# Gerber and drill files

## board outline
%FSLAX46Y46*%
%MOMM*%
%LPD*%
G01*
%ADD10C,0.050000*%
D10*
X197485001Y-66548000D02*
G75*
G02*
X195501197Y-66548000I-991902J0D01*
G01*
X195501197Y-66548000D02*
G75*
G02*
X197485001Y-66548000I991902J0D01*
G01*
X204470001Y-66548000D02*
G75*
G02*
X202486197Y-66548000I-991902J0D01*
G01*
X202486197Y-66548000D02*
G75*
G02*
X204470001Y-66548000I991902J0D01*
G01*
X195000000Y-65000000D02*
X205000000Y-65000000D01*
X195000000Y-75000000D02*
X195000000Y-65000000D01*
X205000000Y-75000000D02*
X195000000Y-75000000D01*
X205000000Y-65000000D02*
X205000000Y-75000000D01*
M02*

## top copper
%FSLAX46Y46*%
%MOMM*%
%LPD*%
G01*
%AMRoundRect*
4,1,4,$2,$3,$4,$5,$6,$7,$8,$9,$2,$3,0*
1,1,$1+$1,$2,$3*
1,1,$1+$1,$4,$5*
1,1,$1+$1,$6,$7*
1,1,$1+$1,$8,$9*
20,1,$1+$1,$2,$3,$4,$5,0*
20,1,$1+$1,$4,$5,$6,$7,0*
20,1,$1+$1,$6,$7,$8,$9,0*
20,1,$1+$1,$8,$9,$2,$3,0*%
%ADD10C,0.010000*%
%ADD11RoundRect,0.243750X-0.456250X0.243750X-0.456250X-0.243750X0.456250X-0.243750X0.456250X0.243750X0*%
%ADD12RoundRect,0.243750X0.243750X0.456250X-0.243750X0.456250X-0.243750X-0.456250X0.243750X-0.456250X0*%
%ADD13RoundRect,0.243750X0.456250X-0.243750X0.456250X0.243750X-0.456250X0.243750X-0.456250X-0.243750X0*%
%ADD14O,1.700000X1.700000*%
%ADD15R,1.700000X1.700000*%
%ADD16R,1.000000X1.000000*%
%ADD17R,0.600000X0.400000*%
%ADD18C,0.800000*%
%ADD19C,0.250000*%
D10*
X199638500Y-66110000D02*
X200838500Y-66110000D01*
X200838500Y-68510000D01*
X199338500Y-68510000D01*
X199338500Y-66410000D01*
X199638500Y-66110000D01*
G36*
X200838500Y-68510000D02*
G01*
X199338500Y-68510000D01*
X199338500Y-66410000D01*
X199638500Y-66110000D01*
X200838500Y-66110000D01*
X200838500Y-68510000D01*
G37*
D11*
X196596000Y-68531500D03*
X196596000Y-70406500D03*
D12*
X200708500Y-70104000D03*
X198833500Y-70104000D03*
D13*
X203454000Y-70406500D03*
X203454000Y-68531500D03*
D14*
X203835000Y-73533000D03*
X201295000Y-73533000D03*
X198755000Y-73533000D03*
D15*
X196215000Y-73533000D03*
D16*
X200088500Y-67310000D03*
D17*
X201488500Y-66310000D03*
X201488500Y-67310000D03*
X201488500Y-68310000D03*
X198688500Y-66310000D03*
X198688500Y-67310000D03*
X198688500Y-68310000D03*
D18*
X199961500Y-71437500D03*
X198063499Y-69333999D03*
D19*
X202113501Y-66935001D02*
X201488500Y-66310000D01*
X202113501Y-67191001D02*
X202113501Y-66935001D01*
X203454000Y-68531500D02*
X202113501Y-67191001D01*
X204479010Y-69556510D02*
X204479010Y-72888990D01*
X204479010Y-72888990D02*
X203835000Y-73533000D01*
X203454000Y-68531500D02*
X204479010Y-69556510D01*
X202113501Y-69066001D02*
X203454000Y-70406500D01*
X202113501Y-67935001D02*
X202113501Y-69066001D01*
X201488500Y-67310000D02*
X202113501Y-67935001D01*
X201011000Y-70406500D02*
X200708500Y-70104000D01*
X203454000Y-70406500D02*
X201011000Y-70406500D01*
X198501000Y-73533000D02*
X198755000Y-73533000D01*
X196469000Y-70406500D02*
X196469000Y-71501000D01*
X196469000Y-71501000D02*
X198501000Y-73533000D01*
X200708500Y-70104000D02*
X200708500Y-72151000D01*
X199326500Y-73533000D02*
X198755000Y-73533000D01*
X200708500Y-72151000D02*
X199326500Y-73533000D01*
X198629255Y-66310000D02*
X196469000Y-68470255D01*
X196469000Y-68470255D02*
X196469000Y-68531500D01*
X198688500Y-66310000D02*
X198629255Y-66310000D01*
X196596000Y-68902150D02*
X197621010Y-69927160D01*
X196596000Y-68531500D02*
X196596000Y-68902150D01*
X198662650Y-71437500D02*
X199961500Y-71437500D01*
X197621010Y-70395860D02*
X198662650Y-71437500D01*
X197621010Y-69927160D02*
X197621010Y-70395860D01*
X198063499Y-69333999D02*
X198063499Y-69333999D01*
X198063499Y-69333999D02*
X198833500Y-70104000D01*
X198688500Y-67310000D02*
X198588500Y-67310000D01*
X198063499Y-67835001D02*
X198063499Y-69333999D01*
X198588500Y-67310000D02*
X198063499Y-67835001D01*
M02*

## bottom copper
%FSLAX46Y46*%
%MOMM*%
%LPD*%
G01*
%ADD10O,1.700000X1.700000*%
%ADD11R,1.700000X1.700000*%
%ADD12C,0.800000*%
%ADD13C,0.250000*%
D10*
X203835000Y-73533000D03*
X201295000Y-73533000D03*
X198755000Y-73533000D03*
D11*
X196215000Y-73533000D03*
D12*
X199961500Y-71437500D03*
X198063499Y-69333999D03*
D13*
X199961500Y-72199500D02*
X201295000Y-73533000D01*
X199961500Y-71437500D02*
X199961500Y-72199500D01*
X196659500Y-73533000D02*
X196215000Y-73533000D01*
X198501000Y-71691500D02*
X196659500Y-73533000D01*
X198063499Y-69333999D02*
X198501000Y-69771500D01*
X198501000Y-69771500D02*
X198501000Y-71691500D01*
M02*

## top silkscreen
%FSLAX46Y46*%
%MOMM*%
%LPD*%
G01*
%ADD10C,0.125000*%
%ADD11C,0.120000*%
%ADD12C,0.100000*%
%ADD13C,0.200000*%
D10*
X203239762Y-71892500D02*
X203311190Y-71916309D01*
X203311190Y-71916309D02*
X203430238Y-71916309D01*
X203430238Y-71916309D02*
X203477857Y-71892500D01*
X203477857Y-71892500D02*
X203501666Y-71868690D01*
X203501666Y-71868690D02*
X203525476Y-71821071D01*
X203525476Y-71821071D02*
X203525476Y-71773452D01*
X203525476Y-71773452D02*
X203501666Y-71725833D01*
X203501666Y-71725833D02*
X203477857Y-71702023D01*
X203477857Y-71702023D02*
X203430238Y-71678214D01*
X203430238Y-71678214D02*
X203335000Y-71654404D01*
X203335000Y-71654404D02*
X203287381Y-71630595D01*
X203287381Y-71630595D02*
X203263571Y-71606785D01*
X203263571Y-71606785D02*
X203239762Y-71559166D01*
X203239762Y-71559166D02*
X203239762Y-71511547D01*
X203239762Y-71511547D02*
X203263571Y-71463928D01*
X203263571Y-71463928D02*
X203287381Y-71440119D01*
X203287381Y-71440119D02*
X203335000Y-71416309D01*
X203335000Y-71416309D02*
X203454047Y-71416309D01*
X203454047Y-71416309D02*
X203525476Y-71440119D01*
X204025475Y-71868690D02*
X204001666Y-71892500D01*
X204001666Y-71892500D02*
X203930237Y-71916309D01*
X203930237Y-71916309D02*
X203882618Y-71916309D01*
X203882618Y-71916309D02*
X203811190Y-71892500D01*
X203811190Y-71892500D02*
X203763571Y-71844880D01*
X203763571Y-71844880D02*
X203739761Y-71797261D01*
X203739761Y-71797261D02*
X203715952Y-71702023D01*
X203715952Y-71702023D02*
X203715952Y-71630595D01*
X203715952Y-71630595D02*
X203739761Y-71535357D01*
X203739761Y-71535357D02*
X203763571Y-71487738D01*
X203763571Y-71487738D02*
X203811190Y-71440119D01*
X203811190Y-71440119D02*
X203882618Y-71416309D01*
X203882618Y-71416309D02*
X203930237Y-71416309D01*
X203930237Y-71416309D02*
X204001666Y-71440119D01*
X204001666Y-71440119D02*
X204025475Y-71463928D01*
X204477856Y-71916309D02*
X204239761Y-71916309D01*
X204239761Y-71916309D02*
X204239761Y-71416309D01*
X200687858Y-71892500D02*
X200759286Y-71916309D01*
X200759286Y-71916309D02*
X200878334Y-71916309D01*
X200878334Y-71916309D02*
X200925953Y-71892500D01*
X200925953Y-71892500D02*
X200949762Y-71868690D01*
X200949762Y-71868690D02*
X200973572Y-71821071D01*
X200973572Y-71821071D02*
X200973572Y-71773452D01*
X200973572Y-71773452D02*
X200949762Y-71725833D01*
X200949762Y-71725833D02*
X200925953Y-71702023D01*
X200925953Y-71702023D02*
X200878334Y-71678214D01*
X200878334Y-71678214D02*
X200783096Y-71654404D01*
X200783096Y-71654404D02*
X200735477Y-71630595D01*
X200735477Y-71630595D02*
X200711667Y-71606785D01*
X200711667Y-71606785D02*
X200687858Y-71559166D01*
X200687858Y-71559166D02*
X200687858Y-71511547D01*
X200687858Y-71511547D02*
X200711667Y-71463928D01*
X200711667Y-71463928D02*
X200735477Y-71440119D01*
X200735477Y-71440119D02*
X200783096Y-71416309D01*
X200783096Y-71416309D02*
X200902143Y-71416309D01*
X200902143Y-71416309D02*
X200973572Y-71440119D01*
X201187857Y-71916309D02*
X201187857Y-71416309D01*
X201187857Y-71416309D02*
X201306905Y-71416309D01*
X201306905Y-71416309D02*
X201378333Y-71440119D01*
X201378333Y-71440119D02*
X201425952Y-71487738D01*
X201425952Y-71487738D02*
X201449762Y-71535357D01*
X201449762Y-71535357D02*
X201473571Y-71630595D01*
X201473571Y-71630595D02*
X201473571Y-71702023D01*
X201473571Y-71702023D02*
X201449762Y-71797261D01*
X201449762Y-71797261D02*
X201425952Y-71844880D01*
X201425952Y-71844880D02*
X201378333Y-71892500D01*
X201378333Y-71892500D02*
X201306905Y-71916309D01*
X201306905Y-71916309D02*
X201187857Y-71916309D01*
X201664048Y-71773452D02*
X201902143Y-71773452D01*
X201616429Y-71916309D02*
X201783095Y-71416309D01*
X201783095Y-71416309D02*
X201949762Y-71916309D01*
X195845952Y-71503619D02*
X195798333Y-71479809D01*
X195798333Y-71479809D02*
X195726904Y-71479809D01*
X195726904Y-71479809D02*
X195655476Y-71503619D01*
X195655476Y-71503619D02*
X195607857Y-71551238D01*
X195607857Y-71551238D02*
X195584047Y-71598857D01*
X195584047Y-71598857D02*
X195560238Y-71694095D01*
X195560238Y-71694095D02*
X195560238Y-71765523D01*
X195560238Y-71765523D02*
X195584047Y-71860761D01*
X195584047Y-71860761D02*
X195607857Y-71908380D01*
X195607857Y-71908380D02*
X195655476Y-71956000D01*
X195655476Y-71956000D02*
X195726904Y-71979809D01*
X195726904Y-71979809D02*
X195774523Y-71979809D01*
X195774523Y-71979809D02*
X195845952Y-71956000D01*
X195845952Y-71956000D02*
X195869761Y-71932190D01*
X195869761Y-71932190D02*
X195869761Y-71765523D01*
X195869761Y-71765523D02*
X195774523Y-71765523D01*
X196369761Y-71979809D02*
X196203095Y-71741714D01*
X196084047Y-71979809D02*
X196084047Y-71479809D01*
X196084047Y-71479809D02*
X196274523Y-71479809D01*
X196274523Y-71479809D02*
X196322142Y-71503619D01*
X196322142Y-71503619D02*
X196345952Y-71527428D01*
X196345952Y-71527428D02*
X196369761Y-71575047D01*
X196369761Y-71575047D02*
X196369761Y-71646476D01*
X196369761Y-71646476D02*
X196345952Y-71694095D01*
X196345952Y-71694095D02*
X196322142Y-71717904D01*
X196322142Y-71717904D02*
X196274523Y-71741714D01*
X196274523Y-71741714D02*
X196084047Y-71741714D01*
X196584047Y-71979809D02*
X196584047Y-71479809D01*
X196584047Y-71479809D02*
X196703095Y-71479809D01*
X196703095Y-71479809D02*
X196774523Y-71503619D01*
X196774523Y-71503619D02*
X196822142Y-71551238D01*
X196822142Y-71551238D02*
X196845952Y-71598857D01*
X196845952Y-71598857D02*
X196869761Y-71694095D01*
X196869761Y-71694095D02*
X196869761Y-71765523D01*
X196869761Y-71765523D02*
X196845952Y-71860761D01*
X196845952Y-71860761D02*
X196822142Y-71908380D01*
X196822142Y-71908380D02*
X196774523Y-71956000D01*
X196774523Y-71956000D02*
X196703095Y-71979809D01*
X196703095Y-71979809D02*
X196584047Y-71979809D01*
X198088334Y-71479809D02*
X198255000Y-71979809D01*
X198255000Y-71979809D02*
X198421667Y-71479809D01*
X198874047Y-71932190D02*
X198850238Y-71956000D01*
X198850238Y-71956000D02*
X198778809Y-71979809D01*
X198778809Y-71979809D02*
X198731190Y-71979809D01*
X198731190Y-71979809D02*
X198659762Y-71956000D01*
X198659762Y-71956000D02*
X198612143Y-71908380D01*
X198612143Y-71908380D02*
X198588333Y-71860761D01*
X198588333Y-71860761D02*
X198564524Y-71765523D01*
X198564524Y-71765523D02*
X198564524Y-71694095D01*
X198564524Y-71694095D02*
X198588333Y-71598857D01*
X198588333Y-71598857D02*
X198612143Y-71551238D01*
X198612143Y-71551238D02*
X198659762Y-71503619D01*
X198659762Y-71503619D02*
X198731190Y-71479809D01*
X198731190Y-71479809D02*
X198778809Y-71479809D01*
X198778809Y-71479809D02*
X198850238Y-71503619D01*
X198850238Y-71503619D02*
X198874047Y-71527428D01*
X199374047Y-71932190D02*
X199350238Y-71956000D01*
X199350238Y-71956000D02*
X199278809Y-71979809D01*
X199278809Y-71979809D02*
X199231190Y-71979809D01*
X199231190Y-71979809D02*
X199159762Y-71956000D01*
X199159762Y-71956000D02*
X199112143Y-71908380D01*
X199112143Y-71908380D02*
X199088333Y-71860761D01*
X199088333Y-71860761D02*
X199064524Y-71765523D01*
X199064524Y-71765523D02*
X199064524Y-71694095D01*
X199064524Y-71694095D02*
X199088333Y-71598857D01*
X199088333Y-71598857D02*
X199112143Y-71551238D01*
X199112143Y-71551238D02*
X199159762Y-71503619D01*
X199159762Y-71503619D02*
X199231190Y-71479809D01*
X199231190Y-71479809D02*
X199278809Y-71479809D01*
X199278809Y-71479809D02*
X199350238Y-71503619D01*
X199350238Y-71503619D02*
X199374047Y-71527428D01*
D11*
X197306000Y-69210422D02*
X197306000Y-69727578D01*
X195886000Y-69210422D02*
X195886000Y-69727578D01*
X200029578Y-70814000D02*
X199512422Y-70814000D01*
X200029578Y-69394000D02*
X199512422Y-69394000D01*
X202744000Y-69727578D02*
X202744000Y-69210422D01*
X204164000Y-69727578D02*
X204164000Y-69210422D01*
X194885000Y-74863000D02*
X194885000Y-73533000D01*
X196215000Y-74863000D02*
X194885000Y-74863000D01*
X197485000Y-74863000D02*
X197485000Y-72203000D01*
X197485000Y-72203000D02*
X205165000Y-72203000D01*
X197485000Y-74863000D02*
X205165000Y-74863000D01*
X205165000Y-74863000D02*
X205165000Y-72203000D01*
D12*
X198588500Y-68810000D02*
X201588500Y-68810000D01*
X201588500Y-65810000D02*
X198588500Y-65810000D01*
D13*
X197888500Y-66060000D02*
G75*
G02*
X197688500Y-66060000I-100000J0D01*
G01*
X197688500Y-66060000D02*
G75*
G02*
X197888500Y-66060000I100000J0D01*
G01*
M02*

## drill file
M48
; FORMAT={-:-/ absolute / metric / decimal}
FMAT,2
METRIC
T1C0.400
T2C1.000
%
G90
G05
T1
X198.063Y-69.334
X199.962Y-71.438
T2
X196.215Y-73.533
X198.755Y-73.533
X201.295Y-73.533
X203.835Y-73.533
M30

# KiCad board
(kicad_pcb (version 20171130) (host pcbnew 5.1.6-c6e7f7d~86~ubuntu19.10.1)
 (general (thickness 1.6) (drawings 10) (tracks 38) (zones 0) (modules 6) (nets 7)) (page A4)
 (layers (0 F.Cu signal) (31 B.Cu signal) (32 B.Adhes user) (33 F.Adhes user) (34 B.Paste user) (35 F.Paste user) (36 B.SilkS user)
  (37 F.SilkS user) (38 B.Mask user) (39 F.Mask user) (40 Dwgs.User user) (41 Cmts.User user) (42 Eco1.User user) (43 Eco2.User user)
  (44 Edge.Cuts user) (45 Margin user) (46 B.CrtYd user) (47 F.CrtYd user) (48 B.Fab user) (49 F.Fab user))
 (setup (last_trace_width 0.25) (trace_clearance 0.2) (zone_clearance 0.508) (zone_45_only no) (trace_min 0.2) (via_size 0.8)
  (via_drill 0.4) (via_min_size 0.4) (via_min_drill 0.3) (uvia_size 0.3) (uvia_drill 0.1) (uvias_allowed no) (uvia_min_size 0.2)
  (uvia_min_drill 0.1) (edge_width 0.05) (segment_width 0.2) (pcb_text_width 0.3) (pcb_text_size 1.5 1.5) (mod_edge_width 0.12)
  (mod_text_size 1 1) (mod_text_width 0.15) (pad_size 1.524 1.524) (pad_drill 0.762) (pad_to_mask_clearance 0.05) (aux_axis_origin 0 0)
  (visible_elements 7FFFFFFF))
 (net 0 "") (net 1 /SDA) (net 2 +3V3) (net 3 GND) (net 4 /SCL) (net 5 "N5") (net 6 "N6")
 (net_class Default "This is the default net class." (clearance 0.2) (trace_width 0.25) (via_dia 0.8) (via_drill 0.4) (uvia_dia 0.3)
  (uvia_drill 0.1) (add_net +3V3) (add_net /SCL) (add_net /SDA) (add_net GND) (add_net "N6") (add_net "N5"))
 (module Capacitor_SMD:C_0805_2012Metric (layer F.Cu) (at 196.596 69.469 270)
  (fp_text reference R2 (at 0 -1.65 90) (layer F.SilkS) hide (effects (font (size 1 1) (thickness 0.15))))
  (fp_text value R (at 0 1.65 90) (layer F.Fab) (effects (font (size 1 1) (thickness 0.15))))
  (fp_line (start -0.258578 -0.71) (end 0.258578 -0.71) (layer F.SilkS) (width 0.12))
  (fp_line (start -0.258578 0.71) (end 0.258578 0.71) (layer F.SilkS) (width 0.12))
  (pad 1 smd roundrect (at -0.9375 0 270) (size 0.975 1.4) (layers F.Cu F.Paste F.Mask) (roundrect_rratio 0.25) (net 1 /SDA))
  (pad 2 smd roundrect (at 0.9375 0 270) (size 0.975 1.4) (layers F.Cu F.Paste F.Mask) (roundrect_rratio 0.25) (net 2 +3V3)))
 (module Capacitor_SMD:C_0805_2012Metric (layer F.Cu) (at 199.771 70.104 180)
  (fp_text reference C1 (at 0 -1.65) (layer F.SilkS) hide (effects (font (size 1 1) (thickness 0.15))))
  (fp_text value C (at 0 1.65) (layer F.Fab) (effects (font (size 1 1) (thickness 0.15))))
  (fp_line (start -0.258578 -0.71) (end 0.258578 -0.71) (layer F.SilkS) (width 0.12))
  (fp_line (start -0.258578 0.71) (end 0.258578 0.71) (layer F.SilkS) (width 0.12))
  (pad 1 smd roundrect (at -0.9375 0 180) (size 0.975 1.4) (layers F.Cu F.Paste F.Mask) (roundrect_rratio 0.25) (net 2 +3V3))
  (pad 2 smd roundrect (at 0.9375 0 180) (size 0.975 1.4) (layers F.Cu F.Paste F.Mask) (roundrect_rratio 0.25) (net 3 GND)))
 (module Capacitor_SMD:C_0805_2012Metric (layer F.Cu) (at 203.454 69.469 90)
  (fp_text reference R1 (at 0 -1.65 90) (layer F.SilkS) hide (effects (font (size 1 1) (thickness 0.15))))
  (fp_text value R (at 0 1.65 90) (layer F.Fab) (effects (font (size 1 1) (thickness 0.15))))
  (fp_line (start -0.258578 -0.71) (end 0.258578 -0.71) (layer F.SilkS) (width 0.12))
  (fp_line (start -0.258578 0.71) (end 0.258578 0.71) (layer F.SilkS) (width 0.12))
  (pad 1 smd roundrect (at -0.9375 0 90) (size 0.975 1.4) (layers F.Cu F.Paste F.Mask) (roundrect_rratio 0.25) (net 2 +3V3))
  (pad 2 smd roundrect (at 0.9375 0 90) (size 0.975 1.4) (layers F.Cu F.Paste F.Mask) (roundrect_rratio 0.25) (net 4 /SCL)))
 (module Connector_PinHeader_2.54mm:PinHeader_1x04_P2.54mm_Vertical (layer F.Cu) (at 196.215 73.533 90)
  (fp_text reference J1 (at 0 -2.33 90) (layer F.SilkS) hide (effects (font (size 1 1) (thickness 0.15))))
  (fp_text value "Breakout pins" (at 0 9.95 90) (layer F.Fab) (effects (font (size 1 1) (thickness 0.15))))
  (fp_line (start -1.33 -1.33) (end 0 -1.33) (layer F.SilkS) (width 0.12))
  (fp_line (start -1.33 0) (end -1.33 -1.33) (layer F.SilkS) (width 0.12))
  (fp_line (start -1.33 1.27) (end 1.33 1.27) (layer F.SilkS) (width 0.12))
  (fp_line (start 1.33 1.27) (end 1.33 8.95) (layer F.SilkS) (width 0.12))
  (fp_line (start -1.33 1.27) (end -1.33 8.95) (layer F.SilkS) (width 0.12))
  (fp_line (start -1.33 8.95) (end 1.33 8.95) (layer F.SilkS) (width 0.12))
  (pad 4 thru_hole oval (at 0 7.62 90) (size 1.7 1.7) (drill 1) (layers *.Cu *.Mask) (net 4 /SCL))
  (pad 3 thru_hole oval (at 0 5.08 90) (size 1.7 1.7) (drill 1) (layers *.Cu *.Mask) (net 1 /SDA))
  (pad 2 thru_hole oval (at 0 2.54 90) (size 1.7 1.7) (drill 1) (layers *.Cu *.Mask) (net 2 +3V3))
  (pad 1 thru_hole rect (at 0 0 90) (size 1.7 1.7) (drill 1) (layers *.Cu *.Mask) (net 3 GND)))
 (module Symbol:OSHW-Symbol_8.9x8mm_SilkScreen (layer B.Cu) (at 200.0885 70.739 180)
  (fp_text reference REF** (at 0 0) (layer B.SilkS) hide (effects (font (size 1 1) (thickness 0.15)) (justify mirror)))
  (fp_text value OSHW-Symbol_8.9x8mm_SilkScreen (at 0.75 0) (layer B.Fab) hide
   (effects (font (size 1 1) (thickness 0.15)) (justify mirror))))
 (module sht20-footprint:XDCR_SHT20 (layer F.Cu) (at 200.0885 67.31)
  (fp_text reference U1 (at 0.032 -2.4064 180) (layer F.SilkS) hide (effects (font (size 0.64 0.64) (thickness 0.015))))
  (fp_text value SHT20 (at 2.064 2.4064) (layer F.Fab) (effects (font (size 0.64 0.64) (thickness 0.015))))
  (fp_line (start -1.5 1.5) (end 1.5 1.5) (layer F.SilkS) (width 0.1))
  (fp_line (start 1.5 -1.5) (end -1.5 -1.5) (layer F.SilkS) (width 0.1))
  (fp_circle (center -2.3 -1.25) (end -2.2 -1.25) (layer F.SilkS) (width 0.2))
  (fp_poly (pts (xy -0.45 -1.2) (xy 0.75 -1.2) (xy 0.75 1.2) (xy -0.75 1.2) (xy -0.75 -0.9)) (layer F.Cu) (width 0.01))
  (pad 7 smd rect (at 0 0) (size 1 1) (layers F.Cu) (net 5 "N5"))
  (pad 6 smd rect (at 1.4 -1) (size 0.6 0.4) (layers F.Cu F.Mask) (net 4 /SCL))
  (pad 5 smd rect (at 1.4 0) (size 0.6 0.4) (layers F.Cu F.Mask) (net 2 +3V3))
  (pad 4 smd rect (at 1.4 1) (size 0.6 0.4) (layers F.Cu F.Mask) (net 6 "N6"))
  (pad 1 smd rect (at -1.4 -1) (size 0.6 0.4) (layers F.Cu F.Mask) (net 1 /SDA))
  (pad 2 smd rect (at -1.4 0) (size 0.6 0.4) (layers F.Cu F.Mask) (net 3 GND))
  (pad 3 smd rect (at -1.4 1) (size 0.6 0.4) (layers F.Cu F.Mask) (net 6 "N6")))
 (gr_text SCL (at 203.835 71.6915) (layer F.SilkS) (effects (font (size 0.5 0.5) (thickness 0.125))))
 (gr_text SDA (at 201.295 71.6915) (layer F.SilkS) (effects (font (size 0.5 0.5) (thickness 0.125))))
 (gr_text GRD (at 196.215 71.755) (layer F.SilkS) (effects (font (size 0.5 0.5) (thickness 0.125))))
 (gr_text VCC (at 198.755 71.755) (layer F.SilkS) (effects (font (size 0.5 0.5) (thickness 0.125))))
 (gr_circle (center 196.493099 66.548) (end 197.255099 67.183) (layer Edge.Cuts) (width 0.05))
 (gr_circle (center 203.478099 66.548) (end 204.240099 67.183) (layer Edge.Cuts) (width 0.05))
 (gr_line (start 195 65) (end 205 65) (layer Edge.Cuts) (width 0.05))
 (gr_line (start 195 75) (end 195 65) (layer Edge.Cuts) (width 0.05))
 (gr_line (start 205 75) (end 195 75) (layer Edge.Cuts) (width 0.05))
 (gr_line (start 205 65) (end 205 75) (layer Edge.Cuts) (width 0.05))
 (segment (start 202.113501 66.935001) (end 201.4885 66.31) (width 0.25) (layer F.Cu) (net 4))
 (segment (start 202.113501 67.191001) (end 202.113501 66.935001) (width 0.25) (layer F.Cu) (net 4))
 (segment (start 203.454 68.5315) (end 202.113501 67.191001) (width 0.25) (layer F.Cu) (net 4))
 (segment (start 204.47901 69.55651) (end 204.47901 72.88899) (width 0.25) (layer F.Cu) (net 4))
 (segment (start 204.47901 72.88899) (end 203.835 73.533) (width 0.25) (layer F.Cu) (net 4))
 (segment (start 203.454 68.5315) (end 204.47901 69.55651) (width 0.25) (layer F.Cu) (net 4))
 (segment (start 202.113501 69.066001) (end 203.454 70.4065) (width 0.25) (layer F.Cu) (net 2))
 (segment (start 202.113501 67.935001) (end 202.113501 69.066001) (width 0.25) (layer F.Cu) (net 2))
 (segment (start 201.4885 67.31) (end 202.113501 67.935001) (width 0.25) (layer F.Cu) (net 2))
 (segment (start 201.011 70.4065) (end 200.7085 70.104) (width 0.25) (layer F.Cu) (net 2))
 (segment (start 203.454 70.4065) (end 201.011 70.4065) (width 0.25) (layer F.Cu) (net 2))
 (segment (start 198.501 73.533) (end 198.755 73.533) (width 0.25) (layer F.Cu) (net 2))
 (segment (start 196.469 70.4065) (end 196.469 71.501) (width 0.25) (layer F.Cu) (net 2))
 (segment (start 196.469 71.501) (end 198.501 73.533) (width 0.25) (layer F.Cu) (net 2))
 (segment (start 200.7085 70.104) (end 200.7085 72.151) (width 0.25) (layer F.Cu) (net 2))
 (segment (start 199.3265 73.533) (end 198.755 73.533) (width 0.25) (layer F.Cu) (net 2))
 (segment (start 200.7085 72.151) (end 199.3265 73.533) (width 0.25) (layer F.Cu) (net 2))
 (via (at 199.9615 71.4375) (size 0.8) (drill 0.4) (layers F.Cu B.Cu) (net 1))
 (segment (start 198.629255 66.31) (end 196.469 68.470255) (width 0.25) (layer F.Cu) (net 1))
 (segment (start 196.469 68.470255) (end 196.469 68.5315) (width 0.25) (layer F.Cu) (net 1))
 (segment (start 198.6885 66.31) (end 198.629255 66.31) (width 0.25) (layer F.Cu) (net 1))
 (segment (start 196.596 68.90215) (end 197.62101 69.92716) (width 0.25) (layer F.Cu) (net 1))
 (segment (start 196.596 68.5315) (end 196.596 68.90215) (width 0.25) (layer F.Cu) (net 1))
 (segment (start 198.66265 71.4375) (end 199.9615 71.4375) (width 0.25) (layer F.Cu) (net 1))
 (segment (start 197.62101 70.39586) (end 198.66265 71.4375) (width 0.25) (layer F.Cu) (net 1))
 (segment (start 197.62101 69.92716) (end 197.62101 70.39586) (width 0.25) (layer F.Cu) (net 1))
 (segment (start 199.9615 72.1995) (end 201.295 73.533) (width 0.25) (layer B.Cu) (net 1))
 (segment (start 199.9615 71.4375) (end 199.9615 72.1995) (width 0.25) (layer B.Cu) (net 1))
 (segment (start 198.063499 69.333999) (end 198.063499 69.333999) (width 0.25) (layer F.Cu) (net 3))
 (segment (start 198.063499 69.333999) (end 198.8335 70.104) (width 0.25) (layer F.Cu) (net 3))
 (via (at 198.063499 69.333999) (size 0.8) (drill 0.4) (layers F.Cu B.Cu) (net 3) (status 1000000))
 (segment (start 198.6885 67.31) (end 198.5885 67.31) (width 0.25) (layer F.Cu) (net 3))
 (segment (start 198.063499 67.835001) (end 198.063499 69.333999) (width 0.25) (layer F.Cu) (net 3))
 (segment (start 198.5885 67.31) (end 198.063499 67.835001) (width 0.25) (layer F.Cu) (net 3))
 (segment (start 196.6595 73.533) (end 196.215 73.533) (width 0.25) (layer B.Cu) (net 3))
 (segment (start 198.501 71.6915) (end 196.6595 73.533) (width 0.25) (layer B.Cu) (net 3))
 (segment (start 198.063499 69.333999) (end 198.501 69.7715) (width 0.25) (layer B.Cu) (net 3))
 (segment (start 198.501 69.7715) (end 198.501 71.6915) (width 0.25) (layer B.Cu) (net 3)))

